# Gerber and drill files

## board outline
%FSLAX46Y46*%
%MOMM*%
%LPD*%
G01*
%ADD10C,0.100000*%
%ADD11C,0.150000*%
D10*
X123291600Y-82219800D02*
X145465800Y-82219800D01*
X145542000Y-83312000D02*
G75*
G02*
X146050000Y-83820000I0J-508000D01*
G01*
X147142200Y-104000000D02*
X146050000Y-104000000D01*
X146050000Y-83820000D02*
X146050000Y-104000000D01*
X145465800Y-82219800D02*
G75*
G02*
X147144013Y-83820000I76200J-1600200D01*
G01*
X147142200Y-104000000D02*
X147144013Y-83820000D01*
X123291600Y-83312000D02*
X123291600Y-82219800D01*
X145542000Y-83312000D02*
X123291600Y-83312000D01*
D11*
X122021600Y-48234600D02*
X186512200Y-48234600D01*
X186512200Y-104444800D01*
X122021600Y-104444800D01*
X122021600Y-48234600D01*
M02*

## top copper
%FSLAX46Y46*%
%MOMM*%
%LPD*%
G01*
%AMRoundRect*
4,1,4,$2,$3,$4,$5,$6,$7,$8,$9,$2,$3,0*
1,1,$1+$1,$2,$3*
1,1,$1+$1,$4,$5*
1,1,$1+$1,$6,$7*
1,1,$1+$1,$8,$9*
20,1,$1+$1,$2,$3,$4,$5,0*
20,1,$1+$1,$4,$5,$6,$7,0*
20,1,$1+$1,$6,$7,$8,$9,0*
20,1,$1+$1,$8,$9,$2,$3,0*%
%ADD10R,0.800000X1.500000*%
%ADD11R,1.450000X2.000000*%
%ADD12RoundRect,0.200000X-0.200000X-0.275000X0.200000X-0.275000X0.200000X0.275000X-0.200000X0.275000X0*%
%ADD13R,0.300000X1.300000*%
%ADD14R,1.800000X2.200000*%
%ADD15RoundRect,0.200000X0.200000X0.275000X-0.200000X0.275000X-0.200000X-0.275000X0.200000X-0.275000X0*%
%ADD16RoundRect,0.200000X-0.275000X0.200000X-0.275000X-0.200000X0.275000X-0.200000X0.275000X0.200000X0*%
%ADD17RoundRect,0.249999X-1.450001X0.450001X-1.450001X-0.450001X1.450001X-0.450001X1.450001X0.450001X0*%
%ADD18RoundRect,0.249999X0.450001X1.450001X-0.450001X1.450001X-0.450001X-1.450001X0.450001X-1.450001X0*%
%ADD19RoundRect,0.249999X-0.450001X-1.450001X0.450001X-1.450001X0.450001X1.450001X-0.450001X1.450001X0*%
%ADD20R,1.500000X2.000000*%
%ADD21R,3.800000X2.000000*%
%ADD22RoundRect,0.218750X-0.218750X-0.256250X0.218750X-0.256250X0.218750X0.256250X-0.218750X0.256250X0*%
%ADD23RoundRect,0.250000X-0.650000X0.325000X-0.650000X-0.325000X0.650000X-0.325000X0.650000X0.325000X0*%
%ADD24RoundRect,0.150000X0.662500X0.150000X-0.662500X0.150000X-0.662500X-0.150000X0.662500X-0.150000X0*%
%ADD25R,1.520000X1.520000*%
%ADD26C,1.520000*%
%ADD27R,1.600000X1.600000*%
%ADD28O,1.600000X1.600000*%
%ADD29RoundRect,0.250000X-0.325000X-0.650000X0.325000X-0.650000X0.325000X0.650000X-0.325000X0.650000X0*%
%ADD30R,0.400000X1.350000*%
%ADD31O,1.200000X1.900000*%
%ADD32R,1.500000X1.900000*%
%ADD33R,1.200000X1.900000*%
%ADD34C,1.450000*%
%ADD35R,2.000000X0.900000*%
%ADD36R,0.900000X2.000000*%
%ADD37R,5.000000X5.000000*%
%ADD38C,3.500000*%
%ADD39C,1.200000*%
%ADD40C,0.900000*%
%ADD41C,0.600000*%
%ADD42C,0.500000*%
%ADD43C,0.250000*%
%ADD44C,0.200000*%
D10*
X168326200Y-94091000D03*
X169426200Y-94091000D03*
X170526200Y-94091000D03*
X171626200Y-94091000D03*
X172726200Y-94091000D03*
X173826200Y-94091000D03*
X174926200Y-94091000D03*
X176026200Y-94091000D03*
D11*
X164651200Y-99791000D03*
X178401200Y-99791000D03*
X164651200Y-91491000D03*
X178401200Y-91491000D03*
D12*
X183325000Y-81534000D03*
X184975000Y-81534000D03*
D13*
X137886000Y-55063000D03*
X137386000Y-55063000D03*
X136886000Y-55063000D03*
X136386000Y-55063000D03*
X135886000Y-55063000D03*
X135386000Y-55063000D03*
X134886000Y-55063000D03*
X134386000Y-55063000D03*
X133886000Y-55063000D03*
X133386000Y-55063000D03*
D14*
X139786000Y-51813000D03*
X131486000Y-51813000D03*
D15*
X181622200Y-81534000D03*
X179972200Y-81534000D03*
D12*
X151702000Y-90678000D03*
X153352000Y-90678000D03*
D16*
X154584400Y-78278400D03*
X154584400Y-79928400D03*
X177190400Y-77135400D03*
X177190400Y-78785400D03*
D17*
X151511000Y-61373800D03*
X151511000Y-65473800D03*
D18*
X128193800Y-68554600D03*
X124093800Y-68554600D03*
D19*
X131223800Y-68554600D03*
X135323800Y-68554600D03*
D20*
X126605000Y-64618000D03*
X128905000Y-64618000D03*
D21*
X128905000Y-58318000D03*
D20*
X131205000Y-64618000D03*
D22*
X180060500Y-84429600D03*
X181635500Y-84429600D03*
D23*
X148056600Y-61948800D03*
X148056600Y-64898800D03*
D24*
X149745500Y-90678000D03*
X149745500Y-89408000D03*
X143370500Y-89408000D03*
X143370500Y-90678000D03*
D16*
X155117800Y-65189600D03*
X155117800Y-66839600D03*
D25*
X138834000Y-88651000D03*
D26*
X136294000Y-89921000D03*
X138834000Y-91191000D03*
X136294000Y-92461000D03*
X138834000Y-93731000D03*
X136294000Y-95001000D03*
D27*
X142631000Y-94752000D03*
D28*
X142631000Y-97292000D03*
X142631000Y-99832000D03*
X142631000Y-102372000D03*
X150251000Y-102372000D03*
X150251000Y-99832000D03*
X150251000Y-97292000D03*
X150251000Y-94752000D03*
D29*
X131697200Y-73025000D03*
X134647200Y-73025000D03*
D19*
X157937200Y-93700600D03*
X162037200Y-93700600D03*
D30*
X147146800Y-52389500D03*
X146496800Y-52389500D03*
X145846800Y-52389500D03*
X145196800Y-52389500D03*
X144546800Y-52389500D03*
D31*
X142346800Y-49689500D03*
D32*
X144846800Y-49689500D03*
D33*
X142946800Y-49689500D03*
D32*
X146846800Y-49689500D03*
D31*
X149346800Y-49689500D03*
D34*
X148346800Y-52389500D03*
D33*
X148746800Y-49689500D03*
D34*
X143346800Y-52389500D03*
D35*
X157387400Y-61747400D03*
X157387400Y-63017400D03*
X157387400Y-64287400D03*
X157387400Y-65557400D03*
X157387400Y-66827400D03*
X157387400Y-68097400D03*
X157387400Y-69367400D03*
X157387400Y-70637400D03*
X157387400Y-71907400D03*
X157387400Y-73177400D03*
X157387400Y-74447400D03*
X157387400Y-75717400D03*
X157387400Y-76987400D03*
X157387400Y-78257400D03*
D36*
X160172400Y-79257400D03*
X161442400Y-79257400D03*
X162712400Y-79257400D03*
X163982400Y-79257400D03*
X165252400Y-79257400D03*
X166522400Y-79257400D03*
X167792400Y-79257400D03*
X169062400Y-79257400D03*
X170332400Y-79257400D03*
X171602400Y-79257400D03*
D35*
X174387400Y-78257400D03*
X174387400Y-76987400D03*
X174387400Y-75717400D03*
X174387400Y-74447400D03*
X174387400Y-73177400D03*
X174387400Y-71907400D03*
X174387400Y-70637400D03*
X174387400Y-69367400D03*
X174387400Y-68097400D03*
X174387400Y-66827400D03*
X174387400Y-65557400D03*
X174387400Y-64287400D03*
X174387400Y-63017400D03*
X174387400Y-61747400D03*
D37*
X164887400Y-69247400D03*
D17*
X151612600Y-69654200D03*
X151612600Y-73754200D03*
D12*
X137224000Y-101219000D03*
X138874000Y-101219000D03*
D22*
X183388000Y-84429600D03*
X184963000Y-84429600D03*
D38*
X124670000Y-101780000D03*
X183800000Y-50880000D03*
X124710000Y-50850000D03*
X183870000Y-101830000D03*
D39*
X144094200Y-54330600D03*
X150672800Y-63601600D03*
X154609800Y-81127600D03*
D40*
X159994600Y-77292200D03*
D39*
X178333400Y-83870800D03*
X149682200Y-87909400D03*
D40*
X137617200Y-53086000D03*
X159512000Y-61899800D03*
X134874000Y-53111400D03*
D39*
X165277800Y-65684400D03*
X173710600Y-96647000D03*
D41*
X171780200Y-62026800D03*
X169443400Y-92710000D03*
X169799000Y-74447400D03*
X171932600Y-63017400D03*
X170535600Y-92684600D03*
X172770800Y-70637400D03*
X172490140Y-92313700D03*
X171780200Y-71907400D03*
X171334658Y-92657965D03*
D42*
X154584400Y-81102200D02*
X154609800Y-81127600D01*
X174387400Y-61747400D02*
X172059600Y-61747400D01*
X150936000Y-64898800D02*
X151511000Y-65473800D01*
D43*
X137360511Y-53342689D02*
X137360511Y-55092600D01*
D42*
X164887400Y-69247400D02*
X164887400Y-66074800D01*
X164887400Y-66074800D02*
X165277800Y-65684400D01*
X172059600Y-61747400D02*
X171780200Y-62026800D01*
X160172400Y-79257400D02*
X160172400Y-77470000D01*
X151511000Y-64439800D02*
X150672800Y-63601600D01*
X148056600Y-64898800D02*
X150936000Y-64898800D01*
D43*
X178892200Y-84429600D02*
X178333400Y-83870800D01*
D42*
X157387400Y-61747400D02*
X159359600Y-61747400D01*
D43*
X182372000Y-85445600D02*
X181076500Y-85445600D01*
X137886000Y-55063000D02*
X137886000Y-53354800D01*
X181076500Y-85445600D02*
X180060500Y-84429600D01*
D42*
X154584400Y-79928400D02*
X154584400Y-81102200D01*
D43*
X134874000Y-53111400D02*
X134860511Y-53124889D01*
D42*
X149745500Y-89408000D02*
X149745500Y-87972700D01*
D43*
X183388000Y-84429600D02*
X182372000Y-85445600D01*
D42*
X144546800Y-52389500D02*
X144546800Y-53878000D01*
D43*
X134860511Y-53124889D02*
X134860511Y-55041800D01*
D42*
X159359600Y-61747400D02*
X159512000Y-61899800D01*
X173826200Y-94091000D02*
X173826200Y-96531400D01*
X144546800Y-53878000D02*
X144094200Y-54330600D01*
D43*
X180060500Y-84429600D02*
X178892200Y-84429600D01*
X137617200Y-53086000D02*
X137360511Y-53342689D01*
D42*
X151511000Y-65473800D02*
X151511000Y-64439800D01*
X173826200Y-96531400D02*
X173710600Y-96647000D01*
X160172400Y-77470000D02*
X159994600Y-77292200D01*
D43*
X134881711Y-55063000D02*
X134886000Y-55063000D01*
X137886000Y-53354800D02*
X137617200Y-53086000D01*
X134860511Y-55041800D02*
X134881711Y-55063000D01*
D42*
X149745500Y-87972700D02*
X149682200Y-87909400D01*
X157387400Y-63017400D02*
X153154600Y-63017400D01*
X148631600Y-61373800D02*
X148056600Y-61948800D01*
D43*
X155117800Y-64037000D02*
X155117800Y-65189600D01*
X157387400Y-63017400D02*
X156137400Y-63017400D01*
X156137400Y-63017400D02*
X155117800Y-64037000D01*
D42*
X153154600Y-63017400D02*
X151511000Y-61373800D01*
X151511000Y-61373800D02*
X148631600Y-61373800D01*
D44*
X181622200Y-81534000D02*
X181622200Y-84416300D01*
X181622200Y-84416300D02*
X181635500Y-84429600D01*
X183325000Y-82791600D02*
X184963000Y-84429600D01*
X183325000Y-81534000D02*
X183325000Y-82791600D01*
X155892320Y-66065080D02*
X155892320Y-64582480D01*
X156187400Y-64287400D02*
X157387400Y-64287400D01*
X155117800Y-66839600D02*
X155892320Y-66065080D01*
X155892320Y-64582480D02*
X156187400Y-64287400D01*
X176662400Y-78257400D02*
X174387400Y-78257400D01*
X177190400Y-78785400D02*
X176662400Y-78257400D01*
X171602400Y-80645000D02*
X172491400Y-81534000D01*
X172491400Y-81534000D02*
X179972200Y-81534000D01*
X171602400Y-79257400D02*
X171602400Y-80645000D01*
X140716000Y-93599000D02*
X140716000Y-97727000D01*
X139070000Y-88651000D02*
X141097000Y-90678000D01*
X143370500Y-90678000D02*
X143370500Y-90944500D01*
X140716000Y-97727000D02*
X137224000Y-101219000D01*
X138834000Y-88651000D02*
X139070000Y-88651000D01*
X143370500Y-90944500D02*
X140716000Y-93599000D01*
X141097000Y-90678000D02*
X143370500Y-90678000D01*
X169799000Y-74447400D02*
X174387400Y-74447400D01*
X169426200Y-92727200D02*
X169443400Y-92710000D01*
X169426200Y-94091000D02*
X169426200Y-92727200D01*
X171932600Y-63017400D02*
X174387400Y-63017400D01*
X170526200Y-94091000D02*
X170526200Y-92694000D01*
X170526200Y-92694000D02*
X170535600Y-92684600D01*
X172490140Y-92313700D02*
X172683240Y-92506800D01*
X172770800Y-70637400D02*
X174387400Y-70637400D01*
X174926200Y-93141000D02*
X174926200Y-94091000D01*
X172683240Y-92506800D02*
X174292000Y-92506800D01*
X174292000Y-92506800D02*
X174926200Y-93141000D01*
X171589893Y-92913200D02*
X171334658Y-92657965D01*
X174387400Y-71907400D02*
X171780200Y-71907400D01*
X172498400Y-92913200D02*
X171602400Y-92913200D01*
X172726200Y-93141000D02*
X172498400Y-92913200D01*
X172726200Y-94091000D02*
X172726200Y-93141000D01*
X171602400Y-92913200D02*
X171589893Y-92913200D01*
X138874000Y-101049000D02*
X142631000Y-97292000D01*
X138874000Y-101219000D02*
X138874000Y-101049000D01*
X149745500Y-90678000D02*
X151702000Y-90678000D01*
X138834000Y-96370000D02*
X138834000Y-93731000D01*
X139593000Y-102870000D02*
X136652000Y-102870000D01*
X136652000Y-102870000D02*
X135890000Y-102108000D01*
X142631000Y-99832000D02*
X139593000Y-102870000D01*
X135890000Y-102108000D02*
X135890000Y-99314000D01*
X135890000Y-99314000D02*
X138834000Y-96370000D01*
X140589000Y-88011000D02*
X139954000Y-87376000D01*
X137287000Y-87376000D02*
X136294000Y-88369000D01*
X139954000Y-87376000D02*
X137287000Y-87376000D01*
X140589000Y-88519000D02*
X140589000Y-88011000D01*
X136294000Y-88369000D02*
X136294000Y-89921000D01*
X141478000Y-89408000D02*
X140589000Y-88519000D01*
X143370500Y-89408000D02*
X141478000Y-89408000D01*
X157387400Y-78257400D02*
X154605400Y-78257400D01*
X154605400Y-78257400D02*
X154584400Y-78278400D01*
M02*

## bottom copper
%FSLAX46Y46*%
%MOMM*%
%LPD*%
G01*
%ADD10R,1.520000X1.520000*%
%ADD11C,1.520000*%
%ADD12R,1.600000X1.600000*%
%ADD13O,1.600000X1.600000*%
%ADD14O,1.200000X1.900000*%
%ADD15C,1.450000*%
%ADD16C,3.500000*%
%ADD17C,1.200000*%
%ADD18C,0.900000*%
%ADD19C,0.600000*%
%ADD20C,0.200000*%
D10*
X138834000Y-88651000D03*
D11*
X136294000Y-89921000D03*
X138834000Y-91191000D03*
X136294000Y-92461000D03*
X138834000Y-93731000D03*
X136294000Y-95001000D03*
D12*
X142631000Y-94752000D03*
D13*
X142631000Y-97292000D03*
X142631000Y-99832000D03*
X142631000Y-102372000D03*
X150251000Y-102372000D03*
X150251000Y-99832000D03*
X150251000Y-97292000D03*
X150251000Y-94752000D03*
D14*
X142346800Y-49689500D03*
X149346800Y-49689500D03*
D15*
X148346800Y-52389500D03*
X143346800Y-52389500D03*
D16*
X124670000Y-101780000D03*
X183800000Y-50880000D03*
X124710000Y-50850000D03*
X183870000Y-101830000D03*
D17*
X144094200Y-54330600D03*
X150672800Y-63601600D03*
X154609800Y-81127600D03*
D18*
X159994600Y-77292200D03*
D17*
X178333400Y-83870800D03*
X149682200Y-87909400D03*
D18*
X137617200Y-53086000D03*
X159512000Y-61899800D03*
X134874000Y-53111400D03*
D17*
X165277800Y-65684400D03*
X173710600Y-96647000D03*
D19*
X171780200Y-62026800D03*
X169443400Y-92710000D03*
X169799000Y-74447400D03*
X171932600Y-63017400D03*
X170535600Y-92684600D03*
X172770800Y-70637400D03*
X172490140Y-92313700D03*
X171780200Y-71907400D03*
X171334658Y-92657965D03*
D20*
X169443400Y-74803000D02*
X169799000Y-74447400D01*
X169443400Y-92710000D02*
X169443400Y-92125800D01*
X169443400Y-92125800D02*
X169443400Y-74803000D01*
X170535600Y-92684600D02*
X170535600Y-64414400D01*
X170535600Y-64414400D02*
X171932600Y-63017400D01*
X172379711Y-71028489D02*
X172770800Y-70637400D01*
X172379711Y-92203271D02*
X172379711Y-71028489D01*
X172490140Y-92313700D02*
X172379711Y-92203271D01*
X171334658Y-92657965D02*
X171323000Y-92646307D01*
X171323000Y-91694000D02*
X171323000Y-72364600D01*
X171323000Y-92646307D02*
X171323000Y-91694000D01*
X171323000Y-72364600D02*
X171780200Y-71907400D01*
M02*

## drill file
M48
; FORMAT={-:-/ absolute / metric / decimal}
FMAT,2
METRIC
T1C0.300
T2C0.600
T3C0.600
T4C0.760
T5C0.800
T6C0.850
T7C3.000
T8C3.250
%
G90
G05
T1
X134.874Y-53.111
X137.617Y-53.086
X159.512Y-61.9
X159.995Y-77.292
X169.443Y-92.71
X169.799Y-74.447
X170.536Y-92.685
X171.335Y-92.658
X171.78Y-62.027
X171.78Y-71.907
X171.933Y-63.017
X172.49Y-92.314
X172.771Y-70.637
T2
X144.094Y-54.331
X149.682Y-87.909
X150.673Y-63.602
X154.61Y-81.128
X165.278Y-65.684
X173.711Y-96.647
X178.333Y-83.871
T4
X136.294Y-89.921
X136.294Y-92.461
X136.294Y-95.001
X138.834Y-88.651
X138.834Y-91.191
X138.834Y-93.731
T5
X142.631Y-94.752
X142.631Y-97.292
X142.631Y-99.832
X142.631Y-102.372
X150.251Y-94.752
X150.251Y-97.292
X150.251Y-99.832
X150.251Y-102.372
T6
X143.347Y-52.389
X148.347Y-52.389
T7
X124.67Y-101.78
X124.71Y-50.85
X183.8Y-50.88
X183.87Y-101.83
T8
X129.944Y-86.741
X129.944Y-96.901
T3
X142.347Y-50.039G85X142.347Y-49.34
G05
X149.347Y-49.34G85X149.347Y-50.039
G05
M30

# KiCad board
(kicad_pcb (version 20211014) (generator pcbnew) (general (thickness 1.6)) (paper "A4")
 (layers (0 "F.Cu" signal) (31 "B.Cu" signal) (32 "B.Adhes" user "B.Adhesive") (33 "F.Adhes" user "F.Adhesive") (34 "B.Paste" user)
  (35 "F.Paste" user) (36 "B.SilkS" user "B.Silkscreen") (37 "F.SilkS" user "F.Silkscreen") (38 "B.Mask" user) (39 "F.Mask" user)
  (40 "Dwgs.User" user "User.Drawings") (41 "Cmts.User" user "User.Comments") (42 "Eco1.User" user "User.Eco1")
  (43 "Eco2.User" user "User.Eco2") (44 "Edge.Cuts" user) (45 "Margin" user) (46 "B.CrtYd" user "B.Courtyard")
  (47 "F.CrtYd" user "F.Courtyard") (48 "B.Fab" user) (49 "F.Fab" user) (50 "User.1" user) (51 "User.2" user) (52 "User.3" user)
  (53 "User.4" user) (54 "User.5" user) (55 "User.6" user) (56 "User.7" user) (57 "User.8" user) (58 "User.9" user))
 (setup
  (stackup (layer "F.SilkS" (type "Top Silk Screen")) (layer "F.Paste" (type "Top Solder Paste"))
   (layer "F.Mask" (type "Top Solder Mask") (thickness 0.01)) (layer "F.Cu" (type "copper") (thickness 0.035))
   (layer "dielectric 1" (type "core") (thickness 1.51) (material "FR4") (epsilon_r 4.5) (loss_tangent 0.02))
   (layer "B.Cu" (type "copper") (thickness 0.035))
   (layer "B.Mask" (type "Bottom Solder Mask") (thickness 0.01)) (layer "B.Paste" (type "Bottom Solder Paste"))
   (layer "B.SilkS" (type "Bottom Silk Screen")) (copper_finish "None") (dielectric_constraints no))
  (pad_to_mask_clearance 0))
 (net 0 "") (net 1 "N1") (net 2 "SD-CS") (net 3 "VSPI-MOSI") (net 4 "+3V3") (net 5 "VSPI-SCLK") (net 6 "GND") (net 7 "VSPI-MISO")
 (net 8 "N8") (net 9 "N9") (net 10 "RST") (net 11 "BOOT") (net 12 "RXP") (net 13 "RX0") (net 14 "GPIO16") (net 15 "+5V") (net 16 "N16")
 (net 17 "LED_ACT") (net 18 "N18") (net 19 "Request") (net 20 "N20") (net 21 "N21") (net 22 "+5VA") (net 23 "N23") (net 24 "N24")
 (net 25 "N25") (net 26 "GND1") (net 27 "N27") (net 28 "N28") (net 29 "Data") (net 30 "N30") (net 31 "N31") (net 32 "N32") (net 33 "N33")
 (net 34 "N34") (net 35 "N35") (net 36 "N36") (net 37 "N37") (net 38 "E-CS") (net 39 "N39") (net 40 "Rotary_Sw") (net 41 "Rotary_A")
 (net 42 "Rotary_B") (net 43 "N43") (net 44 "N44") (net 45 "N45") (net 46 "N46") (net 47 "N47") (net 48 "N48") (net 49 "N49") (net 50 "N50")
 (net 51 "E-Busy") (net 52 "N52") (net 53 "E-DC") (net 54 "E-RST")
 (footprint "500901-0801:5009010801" (layer "F.Cu") (at 171.5262 96.791)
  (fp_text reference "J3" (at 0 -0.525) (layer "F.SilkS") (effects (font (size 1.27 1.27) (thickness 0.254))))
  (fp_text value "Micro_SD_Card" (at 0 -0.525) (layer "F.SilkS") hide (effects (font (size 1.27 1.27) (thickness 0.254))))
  (pad "1" smd rect locked (at -3.2 -2.7) (size 0.8 1.5) (layers "F.Cu" "F.Paste" "F.Mask") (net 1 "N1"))
  (pad "2" smd rect locked (at -2.1 -2.7) (size 0.8 1.5) (layers "F.Cu" "F.Paste" "F.Mask") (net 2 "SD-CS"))
  (pad "3" smd rect locked (at -1 -2.7) (size 0.8 1.5) (layers "F.Cu" "F.Paste" "F.Mask") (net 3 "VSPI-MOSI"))
  (pad "4" smd rect locked (at 0.1 -2.7) (size 0.8 1.5) (layers "F.Cu" "F.Paste" "F.Mask") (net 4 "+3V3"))
  (pad "5" smd rect locked (at 1.2 -2.7) (size 0.8 1.5) (layers "F.Cu" "F.Paste" "F.Mask") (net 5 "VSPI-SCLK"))
  (pad "6" smd rect locked (at 2.3 -2.7) (size 0.8 1.5) (layers "F.Cu" "F.Paste" "F.Mask") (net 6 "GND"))
  (pad "7" smd rect locked (at 3.4 -2.7) (size 0.8 1.5) (layers "F.Cu" "F.Paste" "F.Mask") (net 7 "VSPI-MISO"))
  (pad "8" smd rect locked (at 4.5 -2.7) (size 0.8 1.5) (layers "F.Cu" "F.Paste" "F.Mask") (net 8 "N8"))
  (pad "MP1" smd rect locked (at -6.875 3) (size 1.45 2) (layers "F.Cu" "F.Paste" "F.Mask"))
  (pad "MP2" smd rect locked (at 6.875 3) (size 1.45 2) (layers "F.Cu" "F.Paste" "F.Mask"))
  (pad "MP3" smd rect locked (at -6.875 -5.3) (size 1.45 2) (layers "F.Cu" "F.Paste" "F.Mask"))
  (pad "MP4" smd rect locked (at 6.875 -5.3) (size 1.45 2) (layers "F.Cu" "F.Paste" "F.Mask")))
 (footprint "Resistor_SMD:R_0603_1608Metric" (layer "F.Cu") (at 184.15 81.534)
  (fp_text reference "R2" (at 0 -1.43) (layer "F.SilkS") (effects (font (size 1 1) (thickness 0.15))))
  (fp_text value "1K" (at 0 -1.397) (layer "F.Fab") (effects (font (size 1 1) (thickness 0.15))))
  (pad "1" smd roundrect (at -0.825 0) (size 0.8 0.95) (layers "F.Cu" "F.Paste" "F.Mask") (roundrect_rratio 0.25) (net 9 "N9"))
  (pad "2" smd roundrect (at 0.825 0) (size 0.8 0.95) (layers "F.Cu" "F.Paste" "F.Mask") (roundrect_rratio 0.25) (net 4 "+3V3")))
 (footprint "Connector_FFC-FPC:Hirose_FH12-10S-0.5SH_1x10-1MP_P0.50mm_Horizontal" (layer "F.Cu") (at 135.636 53.213 180)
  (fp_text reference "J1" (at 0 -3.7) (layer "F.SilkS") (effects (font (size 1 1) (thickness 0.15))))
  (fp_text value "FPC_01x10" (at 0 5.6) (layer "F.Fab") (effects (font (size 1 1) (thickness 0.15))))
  (pad "1" smd rect (at -2.25 -1.85 180) (size 0.3 1.3) (layers "F.Cu" "F.Paste" "F.Mask") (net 6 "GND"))
  (pad "2" smd rect (at -1.75 -1.85 180) (size 0.3 1.3) (layers "F.Cu" "F.Paste" "F.Mask") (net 6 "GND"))
  (pad "3" smd rect (at -1.25 -1.85 180) (size 0.3 1.3) (layers "F.Cu" "F.Paste" "F.Mask") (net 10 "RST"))
  (pad "4" smd rect (at -0.75 -1.85 180) (size 0.3 1.3) (layers "F.Cu" "F.Paste" "F.Mask") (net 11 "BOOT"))
  (pad "5" smd rect (at -0.25 -1.85 180) (size 0.3 1.3) (layers "F.Cu" "F.Paste" "F.Mask") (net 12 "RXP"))
  (pad "6" smd rect (at 0.25 -1.85 180) (size 0.3 1.3) (layers "F.Cu" "F.Paste" "F.Mask") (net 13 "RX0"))
  (pad "7" smd rect (at 0.75 -1.85 180) (size 0.3 1.3) (layers "F.Cu" "F.Paste" "F.Mask") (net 6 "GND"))
  (pad "8" smd rect (at 1.25 -1.85 180) (size 0.3 1.3) (layers "F.Cu" "F.Paste" "F.Mask") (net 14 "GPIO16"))
  (pad "9" smd rect (at 1.75 -1.85 180) (size 0.3 1.3) (layers "F.Cu" "F.Paste" "F.Mask") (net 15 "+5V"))
  (pad "10" smd rect (at 2.25 -1.85 180) (size 0.3 1.3) (layers "F.Cu" "F.Paste" "F.Mask") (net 15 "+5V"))
  (pad "MP" smd rect (at -4.15 1.4 180) (size 1.8 2.2) (layers "F.Cu" "F.Paste" "F.Mask"))
  (pad "MP" smd rect (at 4.15 1.4 180) (size 1.8 2.2) (layers "F.Cu" "F.Paste" "F.Mask")))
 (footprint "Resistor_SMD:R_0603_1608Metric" (layer "F.Cu") (at 180.7972 81.534 180)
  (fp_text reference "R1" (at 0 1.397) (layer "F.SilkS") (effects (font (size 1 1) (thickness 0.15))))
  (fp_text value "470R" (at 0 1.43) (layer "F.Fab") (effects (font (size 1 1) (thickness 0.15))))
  (pad "1" smd roundrect (at -0.825 0 180) (size 0.8 0.95) (layers "F.Cu" "F.Paste" "F.Mask") (roundrect_rratio 0.25) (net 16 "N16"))
  (pad "2" smd roundrect (at 0.825 0 180) (size 0.8 0.95) (layers "F.Cu" "F.Paste" "F.Mask") (roundrect_rratio 0.25) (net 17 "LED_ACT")))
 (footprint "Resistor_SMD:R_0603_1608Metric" (layer "F.Cu") (at 152.527 90.678)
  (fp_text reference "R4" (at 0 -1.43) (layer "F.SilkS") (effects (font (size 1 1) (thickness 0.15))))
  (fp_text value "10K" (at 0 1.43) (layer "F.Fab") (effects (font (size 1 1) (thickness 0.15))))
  (pad "1" smd roundrect (at -0.825 0) (size 0.8 0.95) (layers "F.Cu" "F.Paste" "F.Mask") (roundrect_rratio 0.25) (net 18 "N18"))
  (pad "2" smd roundrect (at 0.825 0) (size 0.8 0.95) (layers "F.Cu" "F.Paste" "F.Mask") (roundrect_rratio 0.25) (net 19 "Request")))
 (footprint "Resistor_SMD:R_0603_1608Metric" (layer "F.Cu") (at 154.5844 79.1034 -90)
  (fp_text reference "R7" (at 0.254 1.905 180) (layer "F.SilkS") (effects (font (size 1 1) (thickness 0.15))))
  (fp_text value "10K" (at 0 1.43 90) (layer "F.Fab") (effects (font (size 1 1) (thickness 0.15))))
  (pad "1" smd roundrect (at -0.825 0 270) (size 0.8 0.95) (layers "F.Cu" "F.Paste" "F.Mask") (roundrect_rratio 0.25) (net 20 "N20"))
  (pad "2" smd roundrect (at 0.825 0 270) (size 0.8 0.95) (layers "F.Cu" "F.Paste" "F.Mask") (roundrect_rratio 0.25) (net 6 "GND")))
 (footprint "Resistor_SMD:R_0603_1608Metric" (layer "F.Cu") (at 177.1904 77.9604 -90)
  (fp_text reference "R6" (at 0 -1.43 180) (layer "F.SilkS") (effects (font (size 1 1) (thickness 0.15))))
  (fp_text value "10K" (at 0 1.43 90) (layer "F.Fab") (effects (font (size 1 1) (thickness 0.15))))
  (pad "1" smd roundrect (at -0.825 0 270) (size 0.8 0.95) (layers "F.Cu" "F.Paste" "F.Mask") (roundrect_rratio 0.25) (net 4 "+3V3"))
  (pad "2" smd roundrect (at 0.825 0 270) (size 0.8 0.95) (layers "F.Cu" "F.Paste" "F.Mask") (roundrect_rratio 0.25) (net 11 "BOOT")))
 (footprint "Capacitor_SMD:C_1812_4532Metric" (layer "F.Cu") (at 151.511 63.4238 -90)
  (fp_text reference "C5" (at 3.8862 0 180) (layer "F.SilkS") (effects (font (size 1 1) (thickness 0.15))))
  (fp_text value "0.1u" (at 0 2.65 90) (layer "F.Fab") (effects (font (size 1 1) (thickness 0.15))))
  (pad "1" smd roundrect (at -2.05 0 270) (size 1.4 3.4) (layers "F.Cu" "F.Paste" "F.Mask") (roundrect_rratio 0.178571) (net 4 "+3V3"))
  (pad "2" smd roundrect (at 2.05 0 270) (size 1.4 3.4) (layers "F.Cu" "F.Paste" "F.Mask") (roundrect_rratio 0.178571) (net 6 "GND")))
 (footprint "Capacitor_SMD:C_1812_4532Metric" (layer "F.Cu") (at 126.1438 68.5546 180)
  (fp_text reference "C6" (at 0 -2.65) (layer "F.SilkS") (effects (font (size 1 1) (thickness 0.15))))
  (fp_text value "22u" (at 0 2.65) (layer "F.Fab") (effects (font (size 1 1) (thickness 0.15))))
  (pad "1" smd roundrect (at -2.05 0 180) (size 1.4 3.4) (layers "F.Cu" "F.Paste" "F.Mask") (roundrect_rratio 0.178571) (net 4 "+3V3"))
  (pad "2" smd roundrect (at 2.05 0 180) (size 1.4 3.4) (layers "F.Cu" "F.Paste" "F.Mask") (roundrect_rratio 0.178571) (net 6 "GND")))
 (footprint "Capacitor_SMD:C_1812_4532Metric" (layer "F.Cu") (at 133.2738 68.5546)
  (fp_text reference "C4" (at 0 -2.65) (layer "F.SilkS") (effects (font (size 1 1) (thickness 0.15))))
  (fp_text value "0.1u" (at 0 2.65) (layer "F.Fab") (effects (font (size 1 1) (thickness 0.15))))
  (pad "1" smd roundrect (at -2.05 0) (size 1.4 3.4) (layers "F.Cu" "F.Paste" "F.Mask") (roundrect_rratio 0.178571) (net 15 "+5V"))
  (pad "2" smd roundrect (at 2.05 0) (size 1.4 3.4) (layers "F.Cu" "F.Paste" "F.Mask") (roundrect_rratio 0.178571) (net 6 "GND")))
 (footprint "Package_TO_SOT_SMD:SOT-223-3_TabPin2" (layer "F.Cu") (at 128.905 61.468 90)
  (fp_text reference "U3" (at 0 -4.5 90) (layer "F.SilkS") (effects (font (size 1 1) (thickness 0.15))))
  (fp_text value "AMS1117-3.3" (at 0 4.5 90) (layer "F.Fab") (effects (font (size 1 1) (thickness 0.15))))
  (pad "1" smd rect (at -3.15 -2.3 90) (size 2 1.5) (layers "F.Cu" "F.Paste" "F.Mask") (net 6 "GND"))
  (pad "2" smd rect (at -3.15 0 90) (size 2 1.5) (layers "F.Cu" "F.Paste" "F.Mask") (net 4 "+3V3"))
  (pad "2" smd rect (at 3.15 0 90) (size 2 3.8) (layers "F.Cu" "F.Paste" "F.Mask") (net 4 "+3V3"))
  (pad "3" smd rect (at -3.15 2.3 90) (size 2 1.5) (layers "F.Cu" "F.Paste" "F.Mask") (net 15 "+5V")))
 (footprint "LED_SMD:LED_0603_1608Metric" (layer "F.Cu") (at 180.848 84.4296)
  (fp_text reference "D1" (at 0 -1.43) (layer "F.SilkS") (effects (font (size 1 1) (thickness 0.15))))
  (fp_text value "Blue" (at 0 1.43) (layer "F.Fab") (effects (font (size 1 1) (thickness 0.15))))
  (pad "1" smd roundrect (at -0.7875 0) (size 0.875 0.95) (layers "F.Cu" "F.Paste" "F.Mask") (roundrect_rratio 0.25) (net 6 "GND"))
  (pad "2" smd roundrect (at 0.7875 0) (size 0.875 0.95) (layers "F.Cu" "F.Paste" "F.Mask") (roundrect_rratio 0.25) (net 16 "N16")))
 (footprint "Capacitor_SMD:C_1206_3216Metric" (layer "F.Cu") (at 148.0566 63.4238 -90)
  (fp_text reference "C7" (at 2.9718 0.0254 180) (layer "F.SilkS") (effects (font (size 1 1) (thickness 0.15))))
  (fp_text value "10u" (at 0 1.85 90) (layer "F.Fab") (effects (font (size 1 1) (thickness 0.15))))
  (pad "1" smd roundrect (at -1.475 0 270) (size 1.15 1.8) (layers "F.Cu" "F.Paste" "F.Mask") (roundrect_rratio 0.217391) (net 4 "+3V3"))
  (pad "2" smd roundrect (at 1.475 0 270) (size 1.15 1.8) (layers "F.Cu" "F.Paste" "F.Mask") (roundrect_rratio 0.217391) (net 6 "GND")))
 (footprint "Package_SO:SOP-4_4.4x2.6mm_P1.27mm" (layer "F.Cu") (at 146.558 90.043 180)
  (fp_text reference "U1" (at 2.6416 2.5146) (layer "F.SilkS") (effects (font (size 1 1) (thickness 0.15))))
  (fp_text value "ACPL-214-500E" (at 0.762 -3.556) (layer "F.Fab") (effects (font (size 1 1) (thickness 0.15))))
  (pad "1" smd roundrect (at -3.1875 -0.635 180) (size 1.625 0.6) (layers "F.Cu" "F.Paste" "F.Mask") (roundrect_rratio 0.25) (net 18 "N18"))
  (pad "2" smd roundrect (at -3.1875 0.635 180) (size 1.625 0.6) (layers "F.Cu" "F.Paste" "F.Mask") (roundrect_rratio 0.25) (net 6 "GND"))
  (pad "3" smd roundrect (at 3.1875 0.635 180) (size 1.625 0.6) (layers "F.Cu" "F.Paste" "F.Mask") (roundrect_rratio 0.25) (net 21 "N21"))
  (pad "4" smd roundrect (at 3.1875 -0.635 180) (size 1.625 0.6) (layers "F.Cu" "F.Paste" "F.Mask") (roundrect_rratio 0.25) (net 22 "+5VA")))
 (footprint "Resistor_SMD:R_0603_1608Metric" (layer "F.Cu") (at 155.1178 66.0146 -90)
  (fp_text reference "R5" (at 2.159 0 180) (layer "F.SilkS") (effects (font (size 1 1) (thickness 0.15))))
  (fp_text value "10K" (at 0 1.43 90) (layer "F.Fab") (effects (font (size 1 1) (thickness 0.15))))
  (pad "1" smd roundrect (at -0.825 0 270) (size 0.8 0.95) (layers "F.Cu" "F.Paste" "F.Mask") (roundrect_rratio 0.25) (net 4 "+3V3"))
  (pad "2" smd roundrect (at 0.825 0 270) (size 0.8 0.95) (layers "F.Cu" "F.Paste" "F.Mask") (roundrect_rratio 0.25) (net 10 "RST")))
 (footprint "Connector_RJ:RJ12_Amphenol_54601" (layer "F.Cu") (at 138.834 88.651 -90)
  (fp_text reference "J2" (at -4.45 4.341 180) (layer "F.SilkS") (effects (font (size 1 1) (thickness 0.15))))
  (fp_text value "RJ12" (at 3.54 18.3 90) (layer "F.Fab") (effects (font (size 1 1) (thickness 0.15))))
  (pad "" np_thru_hole circle (at 8.25 8.89 270) (size 3.25 3.25) (drill 3.25) (layers *.Cu *.Mask))
  (pad "" np_thru_hole circle (at -1.91 8.89 270) (size 3.25 3.25) (drill 3.25) (layers *.Cu *.Mask))
  (pad "1" thru_hole rect (at 0 0 270) (size 1.52 1.52) (drill 0.76) (layers *.Cu *.Mask) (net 22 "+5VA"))
  (pad "2" thru_hole circle (at 1.27 2.54 270) (size 1.52 1.52) (drill 0.76) (layers *.Cu *.Mask) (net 21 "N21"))
  (pad "3" thru_hole circle (at 2.54 0 270) (size 1.52 1.52) (drill 0.76) (layers *.Cu *.Mask) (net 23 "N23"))
  (pad "4" thru_hole circle (at 3.81 2.54 270) (size 1.52 1.52) (drill 0.76) (layers *.Cu *.Mask) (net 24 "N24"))
  (pad "5" thru_hole circle (at 5.08 0 270) (size 1.52 1.52) (drill 0.76) (layers *.Cu *.Mask) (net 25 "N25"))
  (pad "6" thru_hole circle (at 6.35 2.54 270) (size 1.52 1.52) (drill 0.76) (layers *.Cu *.Mask) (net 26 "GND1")))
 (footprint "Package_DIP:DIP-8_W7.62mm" (layer "F.Cu") (at 142.631 94.752)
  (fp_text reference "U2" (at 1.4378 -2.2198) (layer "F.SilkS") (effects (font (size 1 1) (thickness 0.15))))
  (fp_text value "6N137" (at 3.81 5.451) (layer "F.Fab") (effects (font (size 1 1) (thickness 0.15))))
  (pad "1" thru_hole rect (at 0 0) (size 1.6 1.6) (drill 0.8) (layers *.Cu *.Mask) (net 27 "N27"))
  (pad "2" thru_hole oval (at 0 2.54) (size 1.6 1.6) (drill 0.8) (layers *.Cu *.Mask) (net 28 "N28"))
  (pad "3" thru_hole oval (at 0 5.08) (size 1.6 1.6) (drill 0.8) (layers *.Cu *.Mask) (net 25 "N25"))
  (pad "4" thru_hole oval (at 0 7.62) (size 1.6 1.6) (drill 0.8) (layers *.Cu *.Mask))
  (pad "5" thru_hole oval (at 7.62 7.62) (size 1.6 1.6) (drill 0.8) (layers *.Cu *.Mask) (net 6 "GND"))
  (pad "6" thru_hole oval (at 7.62 5.08) (size 1.6 1.6) (drill 0.8) (layers *.Cu *.Mask) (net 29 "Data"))
  (pad "7" thru_hole oval (at 7.62 2.54) (size 1.6 1.6) (drill 0.8) (layers *.Cu *.Mask) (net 6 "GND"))
  (pad "8" thru_hole oval (at 7.62 0) (size 1.6 1.6) (drill 0.8) (layers *.Cu *.Mask) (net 4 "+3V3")))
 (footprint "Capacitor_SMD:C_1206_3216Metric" (layer "F.Cu") (at 133.1722 73.025)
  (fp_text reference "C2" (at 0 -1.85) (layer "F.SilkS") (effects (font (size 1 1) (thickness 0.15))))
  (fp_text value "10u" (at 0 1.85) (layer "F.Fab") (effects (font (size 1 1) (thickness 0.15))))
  (pad "1" smd roundrect (at -1.475 0) (size 1.15 1.8) (layers "F.Cu" "F.Paste" "F.Mask") (roundrect_rratio 0.217391) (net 15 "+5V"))
  (pad "2" smd roundrect (at 1.475 0) (size 1.15 1.8) (layers "F.Cu" "F.Paste" "F.Mask") (roundrect_rratio 0.217391) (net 6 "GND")))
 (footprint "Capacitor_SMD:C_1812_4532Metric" (layer "F.Cu") (at 159.9872 93.7006)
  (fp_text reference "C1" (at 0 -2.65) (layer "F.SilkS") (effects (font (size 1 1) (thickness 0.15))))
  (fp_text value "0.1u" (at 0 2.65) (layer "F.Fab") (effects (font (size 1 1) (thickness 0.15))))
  (pad "1" smd roundrect (at -2.05 0) (size 1.4 3.4) (layers "F.Cu" "F.Paste" "F.Mask") (roundrect_rratio 0.178571) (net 4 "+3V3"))
  (pad "2" smd roundrect (at 2.05 0) (size 1.4 3.4) (layers "F.Cu" "F.Paste" "F.Mask") (roundrect_rratio 0.178571) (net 6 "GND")))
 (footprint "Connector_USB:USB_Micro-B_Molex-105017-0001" (layer "F.Cu") (at 145.8468 50.927 180)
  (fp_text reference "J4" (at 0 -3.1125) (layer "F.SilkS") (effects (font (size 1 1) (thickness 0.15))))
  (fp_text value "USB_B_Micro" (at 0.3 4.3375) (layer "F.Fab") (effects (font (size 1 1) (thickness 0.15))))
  (pad "1" smd rect (at -1.3 -1.4625 180) (size 0.4 1.35) (layers "F.Cu" "F.Paste" "F.Mask") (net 15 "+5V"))
  (pad "2" smd rect (at -0.65 -1.4625 180) (size 0.4 1.35) (layers "F.Cu" "F.Paste" "F.Mask") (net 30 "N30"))
  (pad "3" smd rect (at 0 -1.4625 180) (size 0.4 1.35) (layers "F.Cu" "F.Paste" "F.Mask") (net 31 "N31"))
  (pad "4" smd rect (at 0.65 -1.4625 180) (size 0.4 1.35) (layers "F.Cu" "F.Paste" "F.Mask") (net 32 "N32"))
  (pad "5" smd rect (at 1.3 -1.4625 180) (size 0.4 1.35) (layers "F.Cu" "F.Paste" "F.Mask") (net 6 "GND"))
  (pad "6" thru_hole oval (at 3.5 1.2375 180) (size 1.2 1.9) (drill oval 0.6 1.3) (layers *.Cu *.Mask) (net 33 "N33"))
  (pad "6" smd rect (at 1 1.2375 180) (size 1.5 1.9) (layers "F.Cu" "F.Paste" "F.Mask") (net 33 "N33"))
  (pad "6" smd rect (at 2.9 1.2375 180) (size 1.2 1.9) (layers "F.Cu" "F.Mask") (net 33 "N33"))
  (pad "6" smd rect (at -1 1.2375 180) (size 1.5 1.9) (layers "F.Cu" "F.Paste" "F.Mask") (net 33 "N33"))
  (pad "6" thru_hole oval (at -3.5 1.2375) (size 1.2 1.9) (drill oval 0.6 1.3) (layers *.Cu *.Mask) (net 33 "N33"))
  (pad "6" thru_hole circle (at -2.5 -1.4625 180) (size 1.45 1.45) (drill 0.85) (layers *.Cu *.Mask) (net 33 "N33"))
  (pad "6" smd rect (at -2.9 1.2375 180) (size 1.2 1.9) (layers "F.Cu" "F.Mask") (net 33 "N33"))
  (pad "6" thru_hole circle (at 2.5 -1.4625 180) (size 1.45 1.45) (drill 0.85) (layers *.Cu *.Mask) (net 33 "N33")))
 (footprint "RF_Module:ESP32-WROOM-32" (layer "F.Cu") (at 165.8874 70.0024)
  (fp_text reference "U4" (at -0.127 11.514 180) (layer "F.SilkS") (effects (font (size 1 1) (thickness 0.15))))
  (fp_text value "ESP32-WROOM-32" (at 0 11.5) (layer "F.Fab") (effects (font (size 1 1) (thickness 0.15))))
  (pad "1" smd rect (at -8.5 -8.255) (size 2 0.9) (layers "F.Cu" "F.Paste" "F.Mask") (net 6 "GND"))
  (pad "2" smd rect (at -8.5 -6.985) (size 2 0.9) (layers "F.Cu" "F.Paste" "F.Mask") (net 4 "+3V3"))
  (pad "3" smd rect (at -8.5 -5.715) (size 2 0.9) (layers "F.Cu" "F.Paste" "F.Mask") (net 10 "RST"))
  (pad "4" smd rect (at -8.5 -4.445) (size 2 0.9) (layers "F.Cu" "F.Paste" "F.Mask") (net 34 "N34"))
  (pad "5" smd rect (at -8.5 -3.175) (size 2 0.9) (layers "F.Cu" "F.Paste" "F.Mask") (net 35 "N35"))
  (pad "6" smd rect (at -8.5 -1.905) (size 2 0.9) (layers "F.Cu" "F.Paste" "F.Mask") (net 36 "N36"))
  (pad "7" smd rect (at -8.5 -0.635) (size 2 0.9) (layers "F.Cu" "F.Paste" "F.Mask") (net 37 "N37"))
  (pad "8" smd rect (at -8.5 0.635) (size 2 0.9) (layers "F.Cu" "F.Paste" "F.Mask") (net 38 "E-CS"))
  (pad "9" smd rect (at -8.5 1.905) (size 2 0.9) (layers "F.Cu" "F.Paste" "F.Mask") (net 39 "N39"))
  (pad "10" smd rect (at -8.5 3.175) (size 2 0.9) (layers "F.Cu" "F.Paste" "F.Mask") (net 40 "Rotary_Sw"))
  (pad "11" smd rect (at -8.5 4.445) (size 2 0.9) (layers "F.Cu" "F.Paste" "F.Mask") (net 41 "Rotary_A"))
  (pad "12" smd rect (at -8.5 5.715) (size 2 0.9) (layers "F.Cu" "F.Paste" "F.Mask") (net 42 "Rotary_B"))
  (pad "13" smd rect (at -8.5 6.985) (size 2 0.9) (layers "F.Cu" "F.Paste" "F.Mask") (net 29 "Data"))
  (pad "14" smd rect (at -8.5 8.255) (size 2 0.9) (layers "F.Cu" "F.Paste" "F.Mask") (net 20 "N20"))
  (pad "15" smd rect (at -5.715 9.255 90) (size 2 0.9) (layers "F.Cu" "F.Paste" "F.Mask") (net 6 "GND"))
  (pad "16" smd rect (at -4.445 9.255 90) (size 2 0.9) (layers "F.Cu" "F.Paste" "F.Mask") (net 19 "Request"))
  (pad "17" smd rect (at -3.175 9.255 90) (size 2 0.9) (layers "F.Cu" "F.Paste" "F.Mask") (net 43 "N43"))
  (pad "18" smd rect (at -1.905 9.255 90) (size 2 0.9) (layers "F.Cu" "F.Paste" "F.Mask") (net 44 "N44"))
  (pad "19" smd rect (at -0.635 9.255 90) (size 2 0.9) (layers "F.Cu" "F.Paste" "F.Mask") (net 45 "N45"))
  (pad "20" smd rect (at 0.635 9.255 90) (size 2 0.9) (layers "F.Cu" "F.Paste" "F.Mask") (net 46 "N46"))
  (pad "21" smd rect (at 1.905 9.255 90) (size 2 0.9) (layers "F.Cu" "F.Paste" "F.Mask") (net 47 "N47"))
  (pad "22" smd rect (at 3.175 9.255 90) (size 2 0.9) (layers "F.Cu" "F.Paste" "F.Mask") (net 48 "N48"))
  (pad "23" smd rect (at 4.445 9.255 90) (size 2 0.9) (layers "F.Cu" "F.Paste" "F.Mask") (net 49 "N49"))
  (pad "24" smd rect (at 5.715 9.255 90) (size 2 0.9) (layers "F.Cu" "F.Paste" "F.Mask") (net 17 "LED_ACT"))
  (pad "25" smd rect (at 8.5 8.255) (size 2 0.9) (layers "F.Cu" "F.Paste" "F.Mask") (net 11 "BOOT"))
  (pad "26" smd rect (at 8.5 6.985) (size 2 0.9) (layers "F.Cu" "F.Paste" "F.Mask") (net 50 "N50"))
  (pad "27" smd rect (at 8.5 5.715) (size 2 0.9) (layers "F.Cu" "F.Paste" "F.Mask") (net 14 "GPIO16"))
  (pad "28" smd rect (at 8.5 4.445) (size 2 0.9) (layers "F.Cu" "F.Paste" "F.Mask") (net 2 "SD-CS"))
  (pad "29" smd rect (at 8.5 3.175) (size 2 0.9) (layers "F.Cu" "F.Paste" "F.Mask") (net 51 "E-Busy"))
  (pad "30" smd rect (at 8.5 1.905) (size 2 0.9) (layers "F.Cu" "F.Paste" "F.Mask") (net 5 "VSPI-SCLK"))
  (pad "31" smd rect (at 8.5 0.635) (size 2 0.9) (layers "F.Cu" "F.Paste" "F.Mask") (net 7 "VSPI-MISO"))
  (pad "32" smd rect (at 8.5 -0.635) (size 2 0.9) (layers "F.Cu" "F.Paste" "F.Mask") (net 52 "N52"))
  (pad "33" smd rect (at 8.5 -1.905) (size 2 0.9) (layers "F.Cu" "F.Paste" "F.Mask") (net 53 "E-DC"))
  (pad "34" smd rect (at 8.5 -3.175) (size 2 0.9) (layers "F.Cu" "F.Paste" "F.Mask") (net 13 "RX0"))
  (pad "35" smd rect (at 8.5 -4.445) (size 2 0.9) (layers "F.Cu" "F.Paste" "F.Mask") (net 12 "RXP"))
  (pad "36" smd rect (at 8.5 -5.715) (size 2 0.9) (layers "F.Cu" "F.Paste" "F.Mask") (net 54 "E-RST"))
  (pad "37" smd rect (at 8.5 -6.985) (size 2 0.9) (layers "F.Cu" "F.Paste" "F.Mask") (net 3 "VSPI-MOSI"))
  (pad "38" smd rect (at 8.5 -8.255) (size 2 0.9) (layers "F.Cu" "F.Paste" "F.Mask") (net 6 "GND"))
  (pad "39" smd rect (at -1 -0.755) (size 5 5) (layers "F.Cu" "F.Paste" "F.Mask") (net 6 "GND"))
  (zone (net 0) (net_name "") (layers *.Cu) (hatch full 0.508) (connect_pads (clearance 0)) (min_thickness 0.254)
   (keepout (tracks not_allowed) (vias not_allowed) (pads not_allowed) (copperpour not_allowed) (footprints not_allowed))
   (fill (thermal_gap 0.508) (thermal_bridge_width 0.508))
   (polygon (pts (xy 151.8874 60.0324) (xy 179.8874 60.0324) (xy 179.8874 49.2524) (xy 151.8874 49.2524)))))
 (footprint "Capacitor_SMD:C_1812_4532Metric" (layer "F.Cu") (at 151.6126 71.7042 -90)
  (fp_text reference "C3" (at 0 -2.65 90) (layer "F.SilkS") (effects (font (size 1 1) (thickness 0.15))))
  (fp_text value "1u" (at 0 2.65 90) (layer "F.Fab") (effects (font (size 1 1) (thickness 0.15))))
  (pad "1" smd roundrect (at -2.05 0 270) (size 1.4 3.4) (layers "F.Cu" "F.Paste" "F.Mask") (roundrect_rratio 0.178571) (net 10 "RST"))
  (pad "2" smd roundrect (at 2.05 0 270) (size 1.4 3.4) (layers "F.Cu" "F.Paste" "F.Mask") (roundrect_rratio 0.178571) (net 6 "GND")))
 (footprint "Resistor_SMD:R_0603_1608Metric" (layer "F.Cu") (at 138.049 101.219)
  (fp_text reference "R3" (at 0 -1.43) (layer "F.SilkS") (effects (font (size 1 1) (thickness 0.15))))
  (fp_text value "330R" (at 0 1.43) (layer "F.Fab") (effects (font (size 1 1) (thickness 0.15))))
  (pad "1" smd roundrect (at -0.825 0) (size 0.8 0.95) (layers "F.Cu" "F.Paste" "F.Mask") (roundrect_rratio 0.25) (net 22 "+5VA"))
  (pad "2" smd roundrect (at 0.825 0) (size 0.8 0.95) (layers "F.Cu" "F.Paste" "F.Mask") (roundrect_rratio 0.25) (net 28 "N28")))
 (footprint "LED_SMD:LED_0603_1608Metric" (layer "F.Cu") (at 184.1755 84.4296)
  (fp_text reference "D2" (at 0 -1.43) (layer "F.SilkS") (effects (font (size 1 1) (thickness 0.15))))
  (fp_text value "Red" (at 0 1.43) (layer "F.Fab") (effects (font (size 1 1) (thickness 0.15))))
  (pad "1" smd roundrect (at -0.7875 0) (size 0.875 0.95) (layers "F.Cu" "F.Paste" "F.Mask") (roundrect_rratio 0.25) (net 6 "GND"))
  (pad "2" smd roundrect (at 0.7875 0) (size 0.875 0.95) (layers "F.Cu" "F.Paste" "F.Mask") (roundrect_rratio 0.25) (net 9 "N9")))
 (gr_line (start 123.2916 82.2198) (end 145.4658 82.2198) (layer "Edge.Cuts") (width 0.1))
 (gr_arc (start 145.542 83.312) (mid 145.90121 83.46079) (end 146.05 83.82) (layer "Edge.Cuts") (width 0.1))
 (gr_line (start 147.1422 104) (end 146.05 104) (layer "Edge.Cuts") (width 0.1))
 (gr_line (start 146.05 83.82) (end 146.05 104) (layer "Edge.Cuts") (width 0.1))
 (gr_arc (start 145.4658 82.2198) (mid 146.647525 82.660578) (end 147.144013 83.82) (layer "Edge.Cuts") (width 0.1))
 (gr_line (start 147.1422 104) (end 147.144013 83.82) (layer "Edge.Cuts") (width 0.1))
 (gr_line (start 123.2916 83.312) (end 123.2916 82.2198) (layer "Edge.Cuts") (width 0.1))
 (gr_line (start 145.542 83.312) (end 123.2916 83.312) (layer "Edge.Cuts") (width 0.1))
 (gr_rect (start 186.5122 48.2346) (end 122.0216 104.4448) (layer "Edge.Cuts") (width 0.15) (fill none))
 (via (at 124.67 101.78) (size 3.5) (drill 3) (layers "F.Cu" "B.Cu") (free) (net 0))
 (via (at 183.8 50.88) (size 3.5) (drill 3) (layers "F.Cu" "B.Cu") (free) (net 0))
 (via (at 124.71 50.85) (size 3.5) (drill 3) (layers "F.Cu" "B.Cu") (free) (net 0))
 (via (at 183.87 101.83) (size 3.5) (drill 3) (layers "F.Cu" "B.Cu") (free) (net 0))
 (segment (start 154.5844 81.1022) (end 154.6098 81.1276) (width 0.5) (layer "F.Cu") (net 6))
 (segment (start 174.3874 61.7474) (end 172.0596 61.7474) (width 0.5) (layer "F.Cu") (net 6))
 (segment (start 150.936 64.8988) (end 151.511 65.4738) (width 0.5) (layer "F.Cu") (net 6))
 (segment (start 137.360511 53.342689) (end 137.360511 55.0926) (width 0.25) (layer "F.Cu") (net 6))
 (segment (start 164.8874 69.2474) (end 164.8874 66.0748) (width 0.5) (layer "F.Cu") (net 6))
 (segment (start 164.8874 66.0748) (end 165.2778 65.6844) (width 0.5) (layer "F.Cu") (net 6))
 (segment (start 172.0596 61.7474) (end 171.7802 62.0268) (width 0.5) (layer "F.Cu") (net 6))
 (segment (start 160.1724 79.2574) (end 160.1724 77.47) (width 0.5) (layer "F.Cu") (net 6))
 (segment (start 151.511 64.4398) (end 150.6728 63.6016) (width 0.5) (layer "F.Cu") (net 6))
 (segment (start 148.0566 64.8988) (end 150.936 64.8988) (width 0.5) (layer "F.Cu") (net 6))
 (segment (start 178.8922 84.4296) (end 178.3334 83.8708) (width 0.25) (layer "F.Cu") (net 6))
 (segment (start 157.3874 61.7474) (end 159.3596 61.7474) (width 0.5) (layer "F.Cu") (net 6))
 (segment (start 182.372 85.4456) (end 181.0765 85.4456) (width 0.25) (layer "F.Cu") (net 6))
 (segment (start 137.886 55.063) (end 137.886 53.3548) (width 0.25) (layer "F.Cu") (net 6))
 (segment (start 181.0765 85.4456) (end 180.0605 84.4296) (width 0.25) (layer "F.Cu") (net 6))
 (segment (start 154.5844 79.9284) (end 154.5844 81.1022) (width 0.5) (layer "F.Cu") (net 6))
 (segment (start 134.874 53.1114) (end 134.860511 53.124889) (width 0.25) (layer "F.Cu") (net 6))
 (segment (start 149.7455 89.408) (end 149.7455 87.9727) (width 0.5) (layer "F.Cu") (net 6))
 (segment (start 183.388 84.4296) (end 182.372 85.4456) (width 0.25) (layer "F.Cu") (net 6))
 (segment (start 144.5468 52.3895) (end 144.5468 53.878) (width 0.5) (layer "F.Cu") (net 6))
 (segment (start 134.860511 53.124889) (end 134.860511 55.0418) (width 0.25) (layer "F.Cu") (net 6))
 (segment (start 159.3596 61.7474) (end 159.512 61.8998) (width 0.5) (layer "F.Cu") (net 6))
 (segment (start 173.8262 94.091) (end 173.8262 96.5314) (width 0.5) (layer "F.Cu") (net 6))
 (segment (start 144.5468 53.878) (end 144.0942 54.3306) (width 0.5) (layer "F.Cu") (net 6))
 (segment (start 180.0605 84.4296) (end 178.8922 84.4296) (width 0.25) (layer "F.Cu") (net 6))
 (segment (start 137.6172 53.086) (end 137.360511 53.342689) (width 0.25) (layer "F.Cu") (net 6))
 (segment (start 151.511 65.4738) (end 151.511 64.4398) (width 0.5) (layer "F.Cu") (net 6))
 (segment (start 173.8262 96.5314) (end 173.7106 96.647) (width 0.5) (layer "F.Cu") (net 6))
 (segment (start 160.1724 77.47) (end 159.9946 77.2922) (width 0.5) (layer "F.Cu") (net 6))
 (segment (start 134.881711 55.063) (end 134.886 55.063) (width 0.25) (layer "F.Cu") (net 6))
 (segment (start 137.886 53.3548) (end 137.6172 53.086) (width 0.25) (layer "F.Cu") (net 6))
 (segment (start 134.860511 55.0418) (end 134.881711 55.063) (width 0.25) (layer "F.Cu") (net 6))
 (segment (start 149.7455 87.9727) (end 149.6822 87.9094) (width 0.5) (layer "F.Cu") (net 6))
 (via (at 144.0942 54.3306) (size 1.2) (drill 0.6) (layers "F.Cu" "B.Cu") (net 6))
 (via (at 150.6728 63.6016) (size 1.2) (drill 0.6) (layers "F.Cu" "B.Cu") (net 6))
 (via (at 154.6098 81.1276) (size 1.2) (drill 0.6) (layers "F.Cu" "B.Cu") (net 6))
 (via (at 159.9946 77.2922) (size 0.9) (drill 0.3) (layers "F.Cu" "B.Cu") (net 6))
 (via (at 178.3334 83.8708) (size 1.2) (drill 0.6) (layers "F.Cu" "B.Cu") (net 6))
 (via (at 149.6822 87.9094) (size 1.2) (drill 0.6) (layers "F.Cu" "B.Cu") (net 6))
 (via (at 137.6172 53.086) (size 0.9) (drill 0.3) (layers "F.Cu" "B.Cu") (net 6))
 (via (at 159.512 61.8998) (size 0.9) (drill 0.3) (layers "F.Cu" "B.Cu") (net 6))
 (via (at 134.874 53.1114) (size 0.9) (drill 0.3) (layers "F.Cu" "B.Cu") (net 6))
 (via (at 165.2778 65.6844) (size 1.2) (drill 0.6) (layers "F.Cu" "B.Cu") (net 6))
 (via (at 173.7106 96.647) (size 1.2) (drill 0.6) (layers "F.Cu" "B.Cu") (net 6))
 (via (at 171.7802 62.0268) (size 0.6) (drill 0.3) (layers "F.Cu" "B.Cu") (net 6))
 (segment (start 157.3874 63.0174) (end 153.1546 63.0174) (width 0.5) (layer "F.Cu") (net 4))
 (segment (start 148.6316 61.3738) (end 148.0566 61.9488) (width 0.5) (layer "F.Cu") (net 4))
 (segment (start 155.1178 64.037) (end 155.1178 65.1896) (width 0.25) (layer "F.Cu") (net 4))
 (segment (start 157.3874 63.0174) (end 156.1374 63.0174) (width 0.25) (layer "F.Cu") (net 4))
 (segment (start 156.1374 63.0174) (end 155.1178 64.037) (width 0.25) (layer "F.Cu") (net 4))
 (segment (start 153.1546 63.0174) (end 151.511 61.3738) (width 0.5) (layer "F.Cu") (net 4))
 (segment (start 151.511 61.3738) (end 148.6316 61.3738) (width 0.5) (layer "F.Cu") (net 4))
 (segment (start 181.6222 81.534) (end 181.6222 84.4163) (width 0.2) (layer "F.Cu") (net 16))
 (segment (start 181.6222 84.4163) (end 181.6355 84.4296) (width 0.2) (layer "F.Cu") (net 16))
 (segment (start 183.325 82.7916) (end 184.963 84.4296) (width 0.2) (layer "F.Cu") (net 9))
 (segment (start 183.325 81.534) (end 183.325 82.7916) (width 0.2) (layer "F.Cu") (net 9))
 (segment (start 155.89232 66.06508) (end 155.89232 64.58248) (width 0.2) (layer "F.Cu") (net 10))
 (segment (start 156.1874 64.2874) (end 157.3874 64.2874) (width 0.2) (layer "F.Cu") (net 10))
 (segment (start 155.1178 66.8396) (end 155.89232 66.06508) (width 0.2) (layer "F.Cu") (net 10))
 (segment (start 155.89232 64.58248) (end 156.1874 64.2874) (width 0.2) (layer "F.Cu") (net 10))
 (segment (start 176.6624 78.2574) (end 174.3874 78.2574) (width 0.2) (layer "F.Cu") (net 11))
 (segment (start 177.1904 78.7854) (end 176.6624 78.2574) (width 0.2) (layer "F.Cu") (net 11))
 (segment (start 171.6024 80.645) (end 172.4914 81.534) (width 0.2) (layer "F.Cu") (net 17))
 (segment (start 172.4914 81.534) (end 179.9722 81.534) (width 0.2) (layer "F.Cu") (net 17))
 (segment (start 171.6024 79.2574) (end 171.6024 80.645) (width 0.2) (layer "F.Cu") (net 17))
 (segment (start 140.716 93.599) (end 140.716 97.727) (width 0.2) (layer "F.Cu") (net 22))
 (segment (start 139.07 88.651) (end 141.097 90.678) (width 0.2) (layer "F.Cu") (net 22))
 (segment (start 143.3705 90.678) (end 143.3705 90.9445) (width 0.2) (layer "F.Cu") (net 22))
 (segment (start 140.716 97.727) (end 137.224 101.219) (width 0.2) (layer "F.Cu") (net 22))
 (segment (start 138.834 88.651) (end 139.07 88.651) (width 0.2) (layer "F.Cu") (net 22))
 (segment (start 143.3705 90.9445) (end 140.716 93.599) (width 0.2) (layer "F.Cu") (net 22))
 (segment (start 141.097 90.678) (end 143.3705 90.678) (width 0.2) (layer "F.Cu") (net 22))
 (segment (start 169.799 74.4474) (end 174.3874 74.4474) (width 0.2) (layer "F.Cu") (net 2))
 (segment (start 169.4262 92.7272) (end 169.4434 92.71) (width 0.2) (layer "F.Cu") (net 2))
 (segment (start 169.4262 94.091) (end 169.4262 92.7272) (width 0.2) (layer "F.Cu") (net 2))
 (via (at 169.4434 92.71) (size 0.6) (drill 0.3) (layers "F.Cu" "B.Cu") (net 2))
 (via (at 169.799 74.4474) (size 0.6) (drill 0.3) (layers "F.Cu" "B.Cu") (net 2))
 (segment (start 169.4434 74.803) (end 169.799 74.4474) (width 0.2) (layer "B.Cu") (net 2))
 (segment (start 169.4434 92.71) (end 169.4434 92.1258) (width 0.2) (layer "B.Cu") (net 2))
 (segment (start 169.4434 92.1258) (end 169.4434 74.803) (width 0.2) (layer "B.Cu") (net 2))
 (segment (start 171.9326 63.0174) (end 174.3874 63.0174) (width 0.2) (layer "F.Cu") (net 3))
 (segment (start 170.5262 94.091) (end 170.5262 92.694) (width 0.2) (layer "F.Cu") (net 3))
 (segment (start 170.5262 92.694) (end 170.5356 92.6846) (width 0.2) (layer "F.Cu") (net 3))
 (via (at 171.9326 63.0174) (size 0.6) (drill 0.3) (layers "F.Cu" "B.Cu") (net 3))
 (via (at 170.5356 92.6846) (size 0.6) (drill 0.3) (layers "F.Cu" "B.Cu") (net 3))
 (segment (start 170.5356 92.6846) (end 170.5356 64.4144) (width 0.2) (layer "B.Cu") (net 3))
 (segment (start 170.5356 64.4144) (end 171.9326 63.0174) (width 0.2) (layer "B.Cu") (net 3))
 (segment (start 172.49014 92.3137) (end 172.68324 92.5068) (width 0.2) (layer "F.Cu") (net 7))
 (segment (start 172.7708 70.6374) (end 174.3874 70.6374) (width 0.2) (layer "F.Cu") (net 7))
 (segment (start 174.9262 93.141) (end 174.9262 94.091) (width 0.2) (layer "F.Cu") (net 7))
 (segment (start 172.68324 92.5068) (end 174.292 92.5068) (width 0.2) (layer "F.Cu") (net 7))
 (segment (start 174.292 92.5068) (end 174.9262 93.141) (width 0.2) (layer "F.Cu") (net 7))
 (via (at 172.7708 70.6374) (size 0.6) (drill 0.3) (layers "F.Cu" "B.Cu") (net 7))
 (via (at 172.49014 92.3137) (size 0.6) (drill 0.3) (layers "F.Cu" "B.Cu") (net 7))
 (segment (start 172.379711 71.028489) (end 172.7708 70.6374) (width 0.2) (layer "B.Cu") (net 7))
 (segment (start 172.379711 92.203271) (end 172.379711 71.028489) (width 0.2) (layer "B.Cu") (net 7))
 (segment (start 172.49014 92.3137) (end 172.379711 92.203271) (width 0.2) (layer "B.Cu") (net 7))
 (segment (start 171.589893 92.9132) (end 171.334658 92.657965) (width 0.2) (layer "F.Cu") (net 5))
 (segment (start 174.3874 71.9074) (end 171.7802 71.9074) (width 0.2) (layer "F.Cu") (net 5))
 (segment (start 172.4984 92.9132) (end 171.6024 92.9132) (width 0.2) (layer "F.Cu") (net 5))
 (segment (start 172.7262 93.141) (end 172.4984 92.9132) (width 0.2) (layer "F.Cu") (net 5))
 (segment (start 172.7262 94.091) (end 172.7262 93.141) (width 0.2) (layer "F.Cu") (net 5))
 (segment (start 171.6024 92.9132) (end 171.589893 92.9132) (width 0.2) (layer "F.Cu") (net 5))
 (via (at 171.7802 71.9074) (size 0.6) (drill 0.3) (layers "F.Cu" "B.Cu") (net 5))
 (via (at 171.334658 92.657965) (size 0.6) (drill 0.3) (layers "F.Cu" "B.Cu") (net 5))
 (segment (start 171.334658 92.657965) (end 171.323 92.646307) (width 0.2) (layer "B.Cu") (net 5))
 (segment (start 171.323 91.694) (end 171.323 72.3646) (width 0.2) (layer "B.Cu") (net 5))
 (segment (start 171.323 92.646307) (end 171.323 91.694) (width 0.2) (layer "B.Cu") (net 5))
 (segment (start 171.323 72.3646) (end 171.7802 71.9074) (width 0.2) (layer "B.Cu") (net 5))
 (segment (start 138.874 101.049) (end 142.631 97.292) (width 0.2) (layer "F.Cu") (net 28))
 (segment (start 138.874 101.219) (end 138.874 101.049) (width 0.2) (layer "F.Cu") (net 28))
 (segment (start 149.7455 90.678) (end 151.702 90.678) (width 0.2) (layer "F.Cu") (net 18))
 (segment (start 138.834 96.37) (end 138.834 93.731) (width 0.2) (layer "F.Cu") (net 25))
 (segment (start 139.593 102.87) (end 136.652 102.87) (width 0.2) (layer "F.Cu") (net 25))
 (segment (start 136.652 102.87) (end 135.89 102.108) (width 0.2) (layer "F.Cu") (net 25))
 (segment (start 142.631 99.832) (end 139.593 102.87) (width 0.2) (layer "F.Cu") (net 25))
 (segment (start 135.89 102.108) (end 135.89 99.314) (width 0.2) (layer "F.Cu") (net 25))
 (segment (start 135.89 99.314) (end 138.834 96.37) (width 0.2) (layer "F.Cu") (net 25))
 (segment (start 140.589 88.011) (end 139.954 87.376) (width 0.2) (layer "F.Cu") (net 21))
 (segment (start 137.287 87.376) (end 136.294 88.369) (width 0.2) (layer "F.Cu") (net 21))
 (segment (start 139.954 87.376) (end 137.287 87.376) (width 0.2) (layer "F.Cu") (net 21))
 (segment (start 140.589 88.519) (end 140.589 88.011) (width 0.2) (layer "F.Cu") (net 21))
 (segment (start 136.294 88.369) (end 136.294 89.921) (width 0.2) (layer "F.Cu") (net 21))
 (segment (start 141.478 89.408) (end 140.589 88.519) (width 0.2) (layer "F.Cu") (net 21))
 (segment (start 143.3705 89.408) (end 141.478 89.408) (width 0.2) (layer "F.Cu") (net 21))
 (segment (start 157.3874 78.2574) (end 154.6054 78.2574) (width 0.2) (layer "F.Cu") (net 20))
 (segment (start 154.6054 78.2574) (end 154.5844 78.2784) (width 0.2) (layer "F.Cu") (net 20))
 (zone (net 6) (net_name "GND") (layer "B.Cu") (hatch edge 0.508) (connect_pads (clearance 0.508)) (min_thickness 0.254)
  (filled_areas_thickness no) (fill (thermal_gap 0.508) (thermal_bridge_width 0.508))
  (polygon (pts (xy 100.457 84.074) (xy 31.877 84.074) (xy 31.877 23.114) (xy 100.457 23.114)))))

